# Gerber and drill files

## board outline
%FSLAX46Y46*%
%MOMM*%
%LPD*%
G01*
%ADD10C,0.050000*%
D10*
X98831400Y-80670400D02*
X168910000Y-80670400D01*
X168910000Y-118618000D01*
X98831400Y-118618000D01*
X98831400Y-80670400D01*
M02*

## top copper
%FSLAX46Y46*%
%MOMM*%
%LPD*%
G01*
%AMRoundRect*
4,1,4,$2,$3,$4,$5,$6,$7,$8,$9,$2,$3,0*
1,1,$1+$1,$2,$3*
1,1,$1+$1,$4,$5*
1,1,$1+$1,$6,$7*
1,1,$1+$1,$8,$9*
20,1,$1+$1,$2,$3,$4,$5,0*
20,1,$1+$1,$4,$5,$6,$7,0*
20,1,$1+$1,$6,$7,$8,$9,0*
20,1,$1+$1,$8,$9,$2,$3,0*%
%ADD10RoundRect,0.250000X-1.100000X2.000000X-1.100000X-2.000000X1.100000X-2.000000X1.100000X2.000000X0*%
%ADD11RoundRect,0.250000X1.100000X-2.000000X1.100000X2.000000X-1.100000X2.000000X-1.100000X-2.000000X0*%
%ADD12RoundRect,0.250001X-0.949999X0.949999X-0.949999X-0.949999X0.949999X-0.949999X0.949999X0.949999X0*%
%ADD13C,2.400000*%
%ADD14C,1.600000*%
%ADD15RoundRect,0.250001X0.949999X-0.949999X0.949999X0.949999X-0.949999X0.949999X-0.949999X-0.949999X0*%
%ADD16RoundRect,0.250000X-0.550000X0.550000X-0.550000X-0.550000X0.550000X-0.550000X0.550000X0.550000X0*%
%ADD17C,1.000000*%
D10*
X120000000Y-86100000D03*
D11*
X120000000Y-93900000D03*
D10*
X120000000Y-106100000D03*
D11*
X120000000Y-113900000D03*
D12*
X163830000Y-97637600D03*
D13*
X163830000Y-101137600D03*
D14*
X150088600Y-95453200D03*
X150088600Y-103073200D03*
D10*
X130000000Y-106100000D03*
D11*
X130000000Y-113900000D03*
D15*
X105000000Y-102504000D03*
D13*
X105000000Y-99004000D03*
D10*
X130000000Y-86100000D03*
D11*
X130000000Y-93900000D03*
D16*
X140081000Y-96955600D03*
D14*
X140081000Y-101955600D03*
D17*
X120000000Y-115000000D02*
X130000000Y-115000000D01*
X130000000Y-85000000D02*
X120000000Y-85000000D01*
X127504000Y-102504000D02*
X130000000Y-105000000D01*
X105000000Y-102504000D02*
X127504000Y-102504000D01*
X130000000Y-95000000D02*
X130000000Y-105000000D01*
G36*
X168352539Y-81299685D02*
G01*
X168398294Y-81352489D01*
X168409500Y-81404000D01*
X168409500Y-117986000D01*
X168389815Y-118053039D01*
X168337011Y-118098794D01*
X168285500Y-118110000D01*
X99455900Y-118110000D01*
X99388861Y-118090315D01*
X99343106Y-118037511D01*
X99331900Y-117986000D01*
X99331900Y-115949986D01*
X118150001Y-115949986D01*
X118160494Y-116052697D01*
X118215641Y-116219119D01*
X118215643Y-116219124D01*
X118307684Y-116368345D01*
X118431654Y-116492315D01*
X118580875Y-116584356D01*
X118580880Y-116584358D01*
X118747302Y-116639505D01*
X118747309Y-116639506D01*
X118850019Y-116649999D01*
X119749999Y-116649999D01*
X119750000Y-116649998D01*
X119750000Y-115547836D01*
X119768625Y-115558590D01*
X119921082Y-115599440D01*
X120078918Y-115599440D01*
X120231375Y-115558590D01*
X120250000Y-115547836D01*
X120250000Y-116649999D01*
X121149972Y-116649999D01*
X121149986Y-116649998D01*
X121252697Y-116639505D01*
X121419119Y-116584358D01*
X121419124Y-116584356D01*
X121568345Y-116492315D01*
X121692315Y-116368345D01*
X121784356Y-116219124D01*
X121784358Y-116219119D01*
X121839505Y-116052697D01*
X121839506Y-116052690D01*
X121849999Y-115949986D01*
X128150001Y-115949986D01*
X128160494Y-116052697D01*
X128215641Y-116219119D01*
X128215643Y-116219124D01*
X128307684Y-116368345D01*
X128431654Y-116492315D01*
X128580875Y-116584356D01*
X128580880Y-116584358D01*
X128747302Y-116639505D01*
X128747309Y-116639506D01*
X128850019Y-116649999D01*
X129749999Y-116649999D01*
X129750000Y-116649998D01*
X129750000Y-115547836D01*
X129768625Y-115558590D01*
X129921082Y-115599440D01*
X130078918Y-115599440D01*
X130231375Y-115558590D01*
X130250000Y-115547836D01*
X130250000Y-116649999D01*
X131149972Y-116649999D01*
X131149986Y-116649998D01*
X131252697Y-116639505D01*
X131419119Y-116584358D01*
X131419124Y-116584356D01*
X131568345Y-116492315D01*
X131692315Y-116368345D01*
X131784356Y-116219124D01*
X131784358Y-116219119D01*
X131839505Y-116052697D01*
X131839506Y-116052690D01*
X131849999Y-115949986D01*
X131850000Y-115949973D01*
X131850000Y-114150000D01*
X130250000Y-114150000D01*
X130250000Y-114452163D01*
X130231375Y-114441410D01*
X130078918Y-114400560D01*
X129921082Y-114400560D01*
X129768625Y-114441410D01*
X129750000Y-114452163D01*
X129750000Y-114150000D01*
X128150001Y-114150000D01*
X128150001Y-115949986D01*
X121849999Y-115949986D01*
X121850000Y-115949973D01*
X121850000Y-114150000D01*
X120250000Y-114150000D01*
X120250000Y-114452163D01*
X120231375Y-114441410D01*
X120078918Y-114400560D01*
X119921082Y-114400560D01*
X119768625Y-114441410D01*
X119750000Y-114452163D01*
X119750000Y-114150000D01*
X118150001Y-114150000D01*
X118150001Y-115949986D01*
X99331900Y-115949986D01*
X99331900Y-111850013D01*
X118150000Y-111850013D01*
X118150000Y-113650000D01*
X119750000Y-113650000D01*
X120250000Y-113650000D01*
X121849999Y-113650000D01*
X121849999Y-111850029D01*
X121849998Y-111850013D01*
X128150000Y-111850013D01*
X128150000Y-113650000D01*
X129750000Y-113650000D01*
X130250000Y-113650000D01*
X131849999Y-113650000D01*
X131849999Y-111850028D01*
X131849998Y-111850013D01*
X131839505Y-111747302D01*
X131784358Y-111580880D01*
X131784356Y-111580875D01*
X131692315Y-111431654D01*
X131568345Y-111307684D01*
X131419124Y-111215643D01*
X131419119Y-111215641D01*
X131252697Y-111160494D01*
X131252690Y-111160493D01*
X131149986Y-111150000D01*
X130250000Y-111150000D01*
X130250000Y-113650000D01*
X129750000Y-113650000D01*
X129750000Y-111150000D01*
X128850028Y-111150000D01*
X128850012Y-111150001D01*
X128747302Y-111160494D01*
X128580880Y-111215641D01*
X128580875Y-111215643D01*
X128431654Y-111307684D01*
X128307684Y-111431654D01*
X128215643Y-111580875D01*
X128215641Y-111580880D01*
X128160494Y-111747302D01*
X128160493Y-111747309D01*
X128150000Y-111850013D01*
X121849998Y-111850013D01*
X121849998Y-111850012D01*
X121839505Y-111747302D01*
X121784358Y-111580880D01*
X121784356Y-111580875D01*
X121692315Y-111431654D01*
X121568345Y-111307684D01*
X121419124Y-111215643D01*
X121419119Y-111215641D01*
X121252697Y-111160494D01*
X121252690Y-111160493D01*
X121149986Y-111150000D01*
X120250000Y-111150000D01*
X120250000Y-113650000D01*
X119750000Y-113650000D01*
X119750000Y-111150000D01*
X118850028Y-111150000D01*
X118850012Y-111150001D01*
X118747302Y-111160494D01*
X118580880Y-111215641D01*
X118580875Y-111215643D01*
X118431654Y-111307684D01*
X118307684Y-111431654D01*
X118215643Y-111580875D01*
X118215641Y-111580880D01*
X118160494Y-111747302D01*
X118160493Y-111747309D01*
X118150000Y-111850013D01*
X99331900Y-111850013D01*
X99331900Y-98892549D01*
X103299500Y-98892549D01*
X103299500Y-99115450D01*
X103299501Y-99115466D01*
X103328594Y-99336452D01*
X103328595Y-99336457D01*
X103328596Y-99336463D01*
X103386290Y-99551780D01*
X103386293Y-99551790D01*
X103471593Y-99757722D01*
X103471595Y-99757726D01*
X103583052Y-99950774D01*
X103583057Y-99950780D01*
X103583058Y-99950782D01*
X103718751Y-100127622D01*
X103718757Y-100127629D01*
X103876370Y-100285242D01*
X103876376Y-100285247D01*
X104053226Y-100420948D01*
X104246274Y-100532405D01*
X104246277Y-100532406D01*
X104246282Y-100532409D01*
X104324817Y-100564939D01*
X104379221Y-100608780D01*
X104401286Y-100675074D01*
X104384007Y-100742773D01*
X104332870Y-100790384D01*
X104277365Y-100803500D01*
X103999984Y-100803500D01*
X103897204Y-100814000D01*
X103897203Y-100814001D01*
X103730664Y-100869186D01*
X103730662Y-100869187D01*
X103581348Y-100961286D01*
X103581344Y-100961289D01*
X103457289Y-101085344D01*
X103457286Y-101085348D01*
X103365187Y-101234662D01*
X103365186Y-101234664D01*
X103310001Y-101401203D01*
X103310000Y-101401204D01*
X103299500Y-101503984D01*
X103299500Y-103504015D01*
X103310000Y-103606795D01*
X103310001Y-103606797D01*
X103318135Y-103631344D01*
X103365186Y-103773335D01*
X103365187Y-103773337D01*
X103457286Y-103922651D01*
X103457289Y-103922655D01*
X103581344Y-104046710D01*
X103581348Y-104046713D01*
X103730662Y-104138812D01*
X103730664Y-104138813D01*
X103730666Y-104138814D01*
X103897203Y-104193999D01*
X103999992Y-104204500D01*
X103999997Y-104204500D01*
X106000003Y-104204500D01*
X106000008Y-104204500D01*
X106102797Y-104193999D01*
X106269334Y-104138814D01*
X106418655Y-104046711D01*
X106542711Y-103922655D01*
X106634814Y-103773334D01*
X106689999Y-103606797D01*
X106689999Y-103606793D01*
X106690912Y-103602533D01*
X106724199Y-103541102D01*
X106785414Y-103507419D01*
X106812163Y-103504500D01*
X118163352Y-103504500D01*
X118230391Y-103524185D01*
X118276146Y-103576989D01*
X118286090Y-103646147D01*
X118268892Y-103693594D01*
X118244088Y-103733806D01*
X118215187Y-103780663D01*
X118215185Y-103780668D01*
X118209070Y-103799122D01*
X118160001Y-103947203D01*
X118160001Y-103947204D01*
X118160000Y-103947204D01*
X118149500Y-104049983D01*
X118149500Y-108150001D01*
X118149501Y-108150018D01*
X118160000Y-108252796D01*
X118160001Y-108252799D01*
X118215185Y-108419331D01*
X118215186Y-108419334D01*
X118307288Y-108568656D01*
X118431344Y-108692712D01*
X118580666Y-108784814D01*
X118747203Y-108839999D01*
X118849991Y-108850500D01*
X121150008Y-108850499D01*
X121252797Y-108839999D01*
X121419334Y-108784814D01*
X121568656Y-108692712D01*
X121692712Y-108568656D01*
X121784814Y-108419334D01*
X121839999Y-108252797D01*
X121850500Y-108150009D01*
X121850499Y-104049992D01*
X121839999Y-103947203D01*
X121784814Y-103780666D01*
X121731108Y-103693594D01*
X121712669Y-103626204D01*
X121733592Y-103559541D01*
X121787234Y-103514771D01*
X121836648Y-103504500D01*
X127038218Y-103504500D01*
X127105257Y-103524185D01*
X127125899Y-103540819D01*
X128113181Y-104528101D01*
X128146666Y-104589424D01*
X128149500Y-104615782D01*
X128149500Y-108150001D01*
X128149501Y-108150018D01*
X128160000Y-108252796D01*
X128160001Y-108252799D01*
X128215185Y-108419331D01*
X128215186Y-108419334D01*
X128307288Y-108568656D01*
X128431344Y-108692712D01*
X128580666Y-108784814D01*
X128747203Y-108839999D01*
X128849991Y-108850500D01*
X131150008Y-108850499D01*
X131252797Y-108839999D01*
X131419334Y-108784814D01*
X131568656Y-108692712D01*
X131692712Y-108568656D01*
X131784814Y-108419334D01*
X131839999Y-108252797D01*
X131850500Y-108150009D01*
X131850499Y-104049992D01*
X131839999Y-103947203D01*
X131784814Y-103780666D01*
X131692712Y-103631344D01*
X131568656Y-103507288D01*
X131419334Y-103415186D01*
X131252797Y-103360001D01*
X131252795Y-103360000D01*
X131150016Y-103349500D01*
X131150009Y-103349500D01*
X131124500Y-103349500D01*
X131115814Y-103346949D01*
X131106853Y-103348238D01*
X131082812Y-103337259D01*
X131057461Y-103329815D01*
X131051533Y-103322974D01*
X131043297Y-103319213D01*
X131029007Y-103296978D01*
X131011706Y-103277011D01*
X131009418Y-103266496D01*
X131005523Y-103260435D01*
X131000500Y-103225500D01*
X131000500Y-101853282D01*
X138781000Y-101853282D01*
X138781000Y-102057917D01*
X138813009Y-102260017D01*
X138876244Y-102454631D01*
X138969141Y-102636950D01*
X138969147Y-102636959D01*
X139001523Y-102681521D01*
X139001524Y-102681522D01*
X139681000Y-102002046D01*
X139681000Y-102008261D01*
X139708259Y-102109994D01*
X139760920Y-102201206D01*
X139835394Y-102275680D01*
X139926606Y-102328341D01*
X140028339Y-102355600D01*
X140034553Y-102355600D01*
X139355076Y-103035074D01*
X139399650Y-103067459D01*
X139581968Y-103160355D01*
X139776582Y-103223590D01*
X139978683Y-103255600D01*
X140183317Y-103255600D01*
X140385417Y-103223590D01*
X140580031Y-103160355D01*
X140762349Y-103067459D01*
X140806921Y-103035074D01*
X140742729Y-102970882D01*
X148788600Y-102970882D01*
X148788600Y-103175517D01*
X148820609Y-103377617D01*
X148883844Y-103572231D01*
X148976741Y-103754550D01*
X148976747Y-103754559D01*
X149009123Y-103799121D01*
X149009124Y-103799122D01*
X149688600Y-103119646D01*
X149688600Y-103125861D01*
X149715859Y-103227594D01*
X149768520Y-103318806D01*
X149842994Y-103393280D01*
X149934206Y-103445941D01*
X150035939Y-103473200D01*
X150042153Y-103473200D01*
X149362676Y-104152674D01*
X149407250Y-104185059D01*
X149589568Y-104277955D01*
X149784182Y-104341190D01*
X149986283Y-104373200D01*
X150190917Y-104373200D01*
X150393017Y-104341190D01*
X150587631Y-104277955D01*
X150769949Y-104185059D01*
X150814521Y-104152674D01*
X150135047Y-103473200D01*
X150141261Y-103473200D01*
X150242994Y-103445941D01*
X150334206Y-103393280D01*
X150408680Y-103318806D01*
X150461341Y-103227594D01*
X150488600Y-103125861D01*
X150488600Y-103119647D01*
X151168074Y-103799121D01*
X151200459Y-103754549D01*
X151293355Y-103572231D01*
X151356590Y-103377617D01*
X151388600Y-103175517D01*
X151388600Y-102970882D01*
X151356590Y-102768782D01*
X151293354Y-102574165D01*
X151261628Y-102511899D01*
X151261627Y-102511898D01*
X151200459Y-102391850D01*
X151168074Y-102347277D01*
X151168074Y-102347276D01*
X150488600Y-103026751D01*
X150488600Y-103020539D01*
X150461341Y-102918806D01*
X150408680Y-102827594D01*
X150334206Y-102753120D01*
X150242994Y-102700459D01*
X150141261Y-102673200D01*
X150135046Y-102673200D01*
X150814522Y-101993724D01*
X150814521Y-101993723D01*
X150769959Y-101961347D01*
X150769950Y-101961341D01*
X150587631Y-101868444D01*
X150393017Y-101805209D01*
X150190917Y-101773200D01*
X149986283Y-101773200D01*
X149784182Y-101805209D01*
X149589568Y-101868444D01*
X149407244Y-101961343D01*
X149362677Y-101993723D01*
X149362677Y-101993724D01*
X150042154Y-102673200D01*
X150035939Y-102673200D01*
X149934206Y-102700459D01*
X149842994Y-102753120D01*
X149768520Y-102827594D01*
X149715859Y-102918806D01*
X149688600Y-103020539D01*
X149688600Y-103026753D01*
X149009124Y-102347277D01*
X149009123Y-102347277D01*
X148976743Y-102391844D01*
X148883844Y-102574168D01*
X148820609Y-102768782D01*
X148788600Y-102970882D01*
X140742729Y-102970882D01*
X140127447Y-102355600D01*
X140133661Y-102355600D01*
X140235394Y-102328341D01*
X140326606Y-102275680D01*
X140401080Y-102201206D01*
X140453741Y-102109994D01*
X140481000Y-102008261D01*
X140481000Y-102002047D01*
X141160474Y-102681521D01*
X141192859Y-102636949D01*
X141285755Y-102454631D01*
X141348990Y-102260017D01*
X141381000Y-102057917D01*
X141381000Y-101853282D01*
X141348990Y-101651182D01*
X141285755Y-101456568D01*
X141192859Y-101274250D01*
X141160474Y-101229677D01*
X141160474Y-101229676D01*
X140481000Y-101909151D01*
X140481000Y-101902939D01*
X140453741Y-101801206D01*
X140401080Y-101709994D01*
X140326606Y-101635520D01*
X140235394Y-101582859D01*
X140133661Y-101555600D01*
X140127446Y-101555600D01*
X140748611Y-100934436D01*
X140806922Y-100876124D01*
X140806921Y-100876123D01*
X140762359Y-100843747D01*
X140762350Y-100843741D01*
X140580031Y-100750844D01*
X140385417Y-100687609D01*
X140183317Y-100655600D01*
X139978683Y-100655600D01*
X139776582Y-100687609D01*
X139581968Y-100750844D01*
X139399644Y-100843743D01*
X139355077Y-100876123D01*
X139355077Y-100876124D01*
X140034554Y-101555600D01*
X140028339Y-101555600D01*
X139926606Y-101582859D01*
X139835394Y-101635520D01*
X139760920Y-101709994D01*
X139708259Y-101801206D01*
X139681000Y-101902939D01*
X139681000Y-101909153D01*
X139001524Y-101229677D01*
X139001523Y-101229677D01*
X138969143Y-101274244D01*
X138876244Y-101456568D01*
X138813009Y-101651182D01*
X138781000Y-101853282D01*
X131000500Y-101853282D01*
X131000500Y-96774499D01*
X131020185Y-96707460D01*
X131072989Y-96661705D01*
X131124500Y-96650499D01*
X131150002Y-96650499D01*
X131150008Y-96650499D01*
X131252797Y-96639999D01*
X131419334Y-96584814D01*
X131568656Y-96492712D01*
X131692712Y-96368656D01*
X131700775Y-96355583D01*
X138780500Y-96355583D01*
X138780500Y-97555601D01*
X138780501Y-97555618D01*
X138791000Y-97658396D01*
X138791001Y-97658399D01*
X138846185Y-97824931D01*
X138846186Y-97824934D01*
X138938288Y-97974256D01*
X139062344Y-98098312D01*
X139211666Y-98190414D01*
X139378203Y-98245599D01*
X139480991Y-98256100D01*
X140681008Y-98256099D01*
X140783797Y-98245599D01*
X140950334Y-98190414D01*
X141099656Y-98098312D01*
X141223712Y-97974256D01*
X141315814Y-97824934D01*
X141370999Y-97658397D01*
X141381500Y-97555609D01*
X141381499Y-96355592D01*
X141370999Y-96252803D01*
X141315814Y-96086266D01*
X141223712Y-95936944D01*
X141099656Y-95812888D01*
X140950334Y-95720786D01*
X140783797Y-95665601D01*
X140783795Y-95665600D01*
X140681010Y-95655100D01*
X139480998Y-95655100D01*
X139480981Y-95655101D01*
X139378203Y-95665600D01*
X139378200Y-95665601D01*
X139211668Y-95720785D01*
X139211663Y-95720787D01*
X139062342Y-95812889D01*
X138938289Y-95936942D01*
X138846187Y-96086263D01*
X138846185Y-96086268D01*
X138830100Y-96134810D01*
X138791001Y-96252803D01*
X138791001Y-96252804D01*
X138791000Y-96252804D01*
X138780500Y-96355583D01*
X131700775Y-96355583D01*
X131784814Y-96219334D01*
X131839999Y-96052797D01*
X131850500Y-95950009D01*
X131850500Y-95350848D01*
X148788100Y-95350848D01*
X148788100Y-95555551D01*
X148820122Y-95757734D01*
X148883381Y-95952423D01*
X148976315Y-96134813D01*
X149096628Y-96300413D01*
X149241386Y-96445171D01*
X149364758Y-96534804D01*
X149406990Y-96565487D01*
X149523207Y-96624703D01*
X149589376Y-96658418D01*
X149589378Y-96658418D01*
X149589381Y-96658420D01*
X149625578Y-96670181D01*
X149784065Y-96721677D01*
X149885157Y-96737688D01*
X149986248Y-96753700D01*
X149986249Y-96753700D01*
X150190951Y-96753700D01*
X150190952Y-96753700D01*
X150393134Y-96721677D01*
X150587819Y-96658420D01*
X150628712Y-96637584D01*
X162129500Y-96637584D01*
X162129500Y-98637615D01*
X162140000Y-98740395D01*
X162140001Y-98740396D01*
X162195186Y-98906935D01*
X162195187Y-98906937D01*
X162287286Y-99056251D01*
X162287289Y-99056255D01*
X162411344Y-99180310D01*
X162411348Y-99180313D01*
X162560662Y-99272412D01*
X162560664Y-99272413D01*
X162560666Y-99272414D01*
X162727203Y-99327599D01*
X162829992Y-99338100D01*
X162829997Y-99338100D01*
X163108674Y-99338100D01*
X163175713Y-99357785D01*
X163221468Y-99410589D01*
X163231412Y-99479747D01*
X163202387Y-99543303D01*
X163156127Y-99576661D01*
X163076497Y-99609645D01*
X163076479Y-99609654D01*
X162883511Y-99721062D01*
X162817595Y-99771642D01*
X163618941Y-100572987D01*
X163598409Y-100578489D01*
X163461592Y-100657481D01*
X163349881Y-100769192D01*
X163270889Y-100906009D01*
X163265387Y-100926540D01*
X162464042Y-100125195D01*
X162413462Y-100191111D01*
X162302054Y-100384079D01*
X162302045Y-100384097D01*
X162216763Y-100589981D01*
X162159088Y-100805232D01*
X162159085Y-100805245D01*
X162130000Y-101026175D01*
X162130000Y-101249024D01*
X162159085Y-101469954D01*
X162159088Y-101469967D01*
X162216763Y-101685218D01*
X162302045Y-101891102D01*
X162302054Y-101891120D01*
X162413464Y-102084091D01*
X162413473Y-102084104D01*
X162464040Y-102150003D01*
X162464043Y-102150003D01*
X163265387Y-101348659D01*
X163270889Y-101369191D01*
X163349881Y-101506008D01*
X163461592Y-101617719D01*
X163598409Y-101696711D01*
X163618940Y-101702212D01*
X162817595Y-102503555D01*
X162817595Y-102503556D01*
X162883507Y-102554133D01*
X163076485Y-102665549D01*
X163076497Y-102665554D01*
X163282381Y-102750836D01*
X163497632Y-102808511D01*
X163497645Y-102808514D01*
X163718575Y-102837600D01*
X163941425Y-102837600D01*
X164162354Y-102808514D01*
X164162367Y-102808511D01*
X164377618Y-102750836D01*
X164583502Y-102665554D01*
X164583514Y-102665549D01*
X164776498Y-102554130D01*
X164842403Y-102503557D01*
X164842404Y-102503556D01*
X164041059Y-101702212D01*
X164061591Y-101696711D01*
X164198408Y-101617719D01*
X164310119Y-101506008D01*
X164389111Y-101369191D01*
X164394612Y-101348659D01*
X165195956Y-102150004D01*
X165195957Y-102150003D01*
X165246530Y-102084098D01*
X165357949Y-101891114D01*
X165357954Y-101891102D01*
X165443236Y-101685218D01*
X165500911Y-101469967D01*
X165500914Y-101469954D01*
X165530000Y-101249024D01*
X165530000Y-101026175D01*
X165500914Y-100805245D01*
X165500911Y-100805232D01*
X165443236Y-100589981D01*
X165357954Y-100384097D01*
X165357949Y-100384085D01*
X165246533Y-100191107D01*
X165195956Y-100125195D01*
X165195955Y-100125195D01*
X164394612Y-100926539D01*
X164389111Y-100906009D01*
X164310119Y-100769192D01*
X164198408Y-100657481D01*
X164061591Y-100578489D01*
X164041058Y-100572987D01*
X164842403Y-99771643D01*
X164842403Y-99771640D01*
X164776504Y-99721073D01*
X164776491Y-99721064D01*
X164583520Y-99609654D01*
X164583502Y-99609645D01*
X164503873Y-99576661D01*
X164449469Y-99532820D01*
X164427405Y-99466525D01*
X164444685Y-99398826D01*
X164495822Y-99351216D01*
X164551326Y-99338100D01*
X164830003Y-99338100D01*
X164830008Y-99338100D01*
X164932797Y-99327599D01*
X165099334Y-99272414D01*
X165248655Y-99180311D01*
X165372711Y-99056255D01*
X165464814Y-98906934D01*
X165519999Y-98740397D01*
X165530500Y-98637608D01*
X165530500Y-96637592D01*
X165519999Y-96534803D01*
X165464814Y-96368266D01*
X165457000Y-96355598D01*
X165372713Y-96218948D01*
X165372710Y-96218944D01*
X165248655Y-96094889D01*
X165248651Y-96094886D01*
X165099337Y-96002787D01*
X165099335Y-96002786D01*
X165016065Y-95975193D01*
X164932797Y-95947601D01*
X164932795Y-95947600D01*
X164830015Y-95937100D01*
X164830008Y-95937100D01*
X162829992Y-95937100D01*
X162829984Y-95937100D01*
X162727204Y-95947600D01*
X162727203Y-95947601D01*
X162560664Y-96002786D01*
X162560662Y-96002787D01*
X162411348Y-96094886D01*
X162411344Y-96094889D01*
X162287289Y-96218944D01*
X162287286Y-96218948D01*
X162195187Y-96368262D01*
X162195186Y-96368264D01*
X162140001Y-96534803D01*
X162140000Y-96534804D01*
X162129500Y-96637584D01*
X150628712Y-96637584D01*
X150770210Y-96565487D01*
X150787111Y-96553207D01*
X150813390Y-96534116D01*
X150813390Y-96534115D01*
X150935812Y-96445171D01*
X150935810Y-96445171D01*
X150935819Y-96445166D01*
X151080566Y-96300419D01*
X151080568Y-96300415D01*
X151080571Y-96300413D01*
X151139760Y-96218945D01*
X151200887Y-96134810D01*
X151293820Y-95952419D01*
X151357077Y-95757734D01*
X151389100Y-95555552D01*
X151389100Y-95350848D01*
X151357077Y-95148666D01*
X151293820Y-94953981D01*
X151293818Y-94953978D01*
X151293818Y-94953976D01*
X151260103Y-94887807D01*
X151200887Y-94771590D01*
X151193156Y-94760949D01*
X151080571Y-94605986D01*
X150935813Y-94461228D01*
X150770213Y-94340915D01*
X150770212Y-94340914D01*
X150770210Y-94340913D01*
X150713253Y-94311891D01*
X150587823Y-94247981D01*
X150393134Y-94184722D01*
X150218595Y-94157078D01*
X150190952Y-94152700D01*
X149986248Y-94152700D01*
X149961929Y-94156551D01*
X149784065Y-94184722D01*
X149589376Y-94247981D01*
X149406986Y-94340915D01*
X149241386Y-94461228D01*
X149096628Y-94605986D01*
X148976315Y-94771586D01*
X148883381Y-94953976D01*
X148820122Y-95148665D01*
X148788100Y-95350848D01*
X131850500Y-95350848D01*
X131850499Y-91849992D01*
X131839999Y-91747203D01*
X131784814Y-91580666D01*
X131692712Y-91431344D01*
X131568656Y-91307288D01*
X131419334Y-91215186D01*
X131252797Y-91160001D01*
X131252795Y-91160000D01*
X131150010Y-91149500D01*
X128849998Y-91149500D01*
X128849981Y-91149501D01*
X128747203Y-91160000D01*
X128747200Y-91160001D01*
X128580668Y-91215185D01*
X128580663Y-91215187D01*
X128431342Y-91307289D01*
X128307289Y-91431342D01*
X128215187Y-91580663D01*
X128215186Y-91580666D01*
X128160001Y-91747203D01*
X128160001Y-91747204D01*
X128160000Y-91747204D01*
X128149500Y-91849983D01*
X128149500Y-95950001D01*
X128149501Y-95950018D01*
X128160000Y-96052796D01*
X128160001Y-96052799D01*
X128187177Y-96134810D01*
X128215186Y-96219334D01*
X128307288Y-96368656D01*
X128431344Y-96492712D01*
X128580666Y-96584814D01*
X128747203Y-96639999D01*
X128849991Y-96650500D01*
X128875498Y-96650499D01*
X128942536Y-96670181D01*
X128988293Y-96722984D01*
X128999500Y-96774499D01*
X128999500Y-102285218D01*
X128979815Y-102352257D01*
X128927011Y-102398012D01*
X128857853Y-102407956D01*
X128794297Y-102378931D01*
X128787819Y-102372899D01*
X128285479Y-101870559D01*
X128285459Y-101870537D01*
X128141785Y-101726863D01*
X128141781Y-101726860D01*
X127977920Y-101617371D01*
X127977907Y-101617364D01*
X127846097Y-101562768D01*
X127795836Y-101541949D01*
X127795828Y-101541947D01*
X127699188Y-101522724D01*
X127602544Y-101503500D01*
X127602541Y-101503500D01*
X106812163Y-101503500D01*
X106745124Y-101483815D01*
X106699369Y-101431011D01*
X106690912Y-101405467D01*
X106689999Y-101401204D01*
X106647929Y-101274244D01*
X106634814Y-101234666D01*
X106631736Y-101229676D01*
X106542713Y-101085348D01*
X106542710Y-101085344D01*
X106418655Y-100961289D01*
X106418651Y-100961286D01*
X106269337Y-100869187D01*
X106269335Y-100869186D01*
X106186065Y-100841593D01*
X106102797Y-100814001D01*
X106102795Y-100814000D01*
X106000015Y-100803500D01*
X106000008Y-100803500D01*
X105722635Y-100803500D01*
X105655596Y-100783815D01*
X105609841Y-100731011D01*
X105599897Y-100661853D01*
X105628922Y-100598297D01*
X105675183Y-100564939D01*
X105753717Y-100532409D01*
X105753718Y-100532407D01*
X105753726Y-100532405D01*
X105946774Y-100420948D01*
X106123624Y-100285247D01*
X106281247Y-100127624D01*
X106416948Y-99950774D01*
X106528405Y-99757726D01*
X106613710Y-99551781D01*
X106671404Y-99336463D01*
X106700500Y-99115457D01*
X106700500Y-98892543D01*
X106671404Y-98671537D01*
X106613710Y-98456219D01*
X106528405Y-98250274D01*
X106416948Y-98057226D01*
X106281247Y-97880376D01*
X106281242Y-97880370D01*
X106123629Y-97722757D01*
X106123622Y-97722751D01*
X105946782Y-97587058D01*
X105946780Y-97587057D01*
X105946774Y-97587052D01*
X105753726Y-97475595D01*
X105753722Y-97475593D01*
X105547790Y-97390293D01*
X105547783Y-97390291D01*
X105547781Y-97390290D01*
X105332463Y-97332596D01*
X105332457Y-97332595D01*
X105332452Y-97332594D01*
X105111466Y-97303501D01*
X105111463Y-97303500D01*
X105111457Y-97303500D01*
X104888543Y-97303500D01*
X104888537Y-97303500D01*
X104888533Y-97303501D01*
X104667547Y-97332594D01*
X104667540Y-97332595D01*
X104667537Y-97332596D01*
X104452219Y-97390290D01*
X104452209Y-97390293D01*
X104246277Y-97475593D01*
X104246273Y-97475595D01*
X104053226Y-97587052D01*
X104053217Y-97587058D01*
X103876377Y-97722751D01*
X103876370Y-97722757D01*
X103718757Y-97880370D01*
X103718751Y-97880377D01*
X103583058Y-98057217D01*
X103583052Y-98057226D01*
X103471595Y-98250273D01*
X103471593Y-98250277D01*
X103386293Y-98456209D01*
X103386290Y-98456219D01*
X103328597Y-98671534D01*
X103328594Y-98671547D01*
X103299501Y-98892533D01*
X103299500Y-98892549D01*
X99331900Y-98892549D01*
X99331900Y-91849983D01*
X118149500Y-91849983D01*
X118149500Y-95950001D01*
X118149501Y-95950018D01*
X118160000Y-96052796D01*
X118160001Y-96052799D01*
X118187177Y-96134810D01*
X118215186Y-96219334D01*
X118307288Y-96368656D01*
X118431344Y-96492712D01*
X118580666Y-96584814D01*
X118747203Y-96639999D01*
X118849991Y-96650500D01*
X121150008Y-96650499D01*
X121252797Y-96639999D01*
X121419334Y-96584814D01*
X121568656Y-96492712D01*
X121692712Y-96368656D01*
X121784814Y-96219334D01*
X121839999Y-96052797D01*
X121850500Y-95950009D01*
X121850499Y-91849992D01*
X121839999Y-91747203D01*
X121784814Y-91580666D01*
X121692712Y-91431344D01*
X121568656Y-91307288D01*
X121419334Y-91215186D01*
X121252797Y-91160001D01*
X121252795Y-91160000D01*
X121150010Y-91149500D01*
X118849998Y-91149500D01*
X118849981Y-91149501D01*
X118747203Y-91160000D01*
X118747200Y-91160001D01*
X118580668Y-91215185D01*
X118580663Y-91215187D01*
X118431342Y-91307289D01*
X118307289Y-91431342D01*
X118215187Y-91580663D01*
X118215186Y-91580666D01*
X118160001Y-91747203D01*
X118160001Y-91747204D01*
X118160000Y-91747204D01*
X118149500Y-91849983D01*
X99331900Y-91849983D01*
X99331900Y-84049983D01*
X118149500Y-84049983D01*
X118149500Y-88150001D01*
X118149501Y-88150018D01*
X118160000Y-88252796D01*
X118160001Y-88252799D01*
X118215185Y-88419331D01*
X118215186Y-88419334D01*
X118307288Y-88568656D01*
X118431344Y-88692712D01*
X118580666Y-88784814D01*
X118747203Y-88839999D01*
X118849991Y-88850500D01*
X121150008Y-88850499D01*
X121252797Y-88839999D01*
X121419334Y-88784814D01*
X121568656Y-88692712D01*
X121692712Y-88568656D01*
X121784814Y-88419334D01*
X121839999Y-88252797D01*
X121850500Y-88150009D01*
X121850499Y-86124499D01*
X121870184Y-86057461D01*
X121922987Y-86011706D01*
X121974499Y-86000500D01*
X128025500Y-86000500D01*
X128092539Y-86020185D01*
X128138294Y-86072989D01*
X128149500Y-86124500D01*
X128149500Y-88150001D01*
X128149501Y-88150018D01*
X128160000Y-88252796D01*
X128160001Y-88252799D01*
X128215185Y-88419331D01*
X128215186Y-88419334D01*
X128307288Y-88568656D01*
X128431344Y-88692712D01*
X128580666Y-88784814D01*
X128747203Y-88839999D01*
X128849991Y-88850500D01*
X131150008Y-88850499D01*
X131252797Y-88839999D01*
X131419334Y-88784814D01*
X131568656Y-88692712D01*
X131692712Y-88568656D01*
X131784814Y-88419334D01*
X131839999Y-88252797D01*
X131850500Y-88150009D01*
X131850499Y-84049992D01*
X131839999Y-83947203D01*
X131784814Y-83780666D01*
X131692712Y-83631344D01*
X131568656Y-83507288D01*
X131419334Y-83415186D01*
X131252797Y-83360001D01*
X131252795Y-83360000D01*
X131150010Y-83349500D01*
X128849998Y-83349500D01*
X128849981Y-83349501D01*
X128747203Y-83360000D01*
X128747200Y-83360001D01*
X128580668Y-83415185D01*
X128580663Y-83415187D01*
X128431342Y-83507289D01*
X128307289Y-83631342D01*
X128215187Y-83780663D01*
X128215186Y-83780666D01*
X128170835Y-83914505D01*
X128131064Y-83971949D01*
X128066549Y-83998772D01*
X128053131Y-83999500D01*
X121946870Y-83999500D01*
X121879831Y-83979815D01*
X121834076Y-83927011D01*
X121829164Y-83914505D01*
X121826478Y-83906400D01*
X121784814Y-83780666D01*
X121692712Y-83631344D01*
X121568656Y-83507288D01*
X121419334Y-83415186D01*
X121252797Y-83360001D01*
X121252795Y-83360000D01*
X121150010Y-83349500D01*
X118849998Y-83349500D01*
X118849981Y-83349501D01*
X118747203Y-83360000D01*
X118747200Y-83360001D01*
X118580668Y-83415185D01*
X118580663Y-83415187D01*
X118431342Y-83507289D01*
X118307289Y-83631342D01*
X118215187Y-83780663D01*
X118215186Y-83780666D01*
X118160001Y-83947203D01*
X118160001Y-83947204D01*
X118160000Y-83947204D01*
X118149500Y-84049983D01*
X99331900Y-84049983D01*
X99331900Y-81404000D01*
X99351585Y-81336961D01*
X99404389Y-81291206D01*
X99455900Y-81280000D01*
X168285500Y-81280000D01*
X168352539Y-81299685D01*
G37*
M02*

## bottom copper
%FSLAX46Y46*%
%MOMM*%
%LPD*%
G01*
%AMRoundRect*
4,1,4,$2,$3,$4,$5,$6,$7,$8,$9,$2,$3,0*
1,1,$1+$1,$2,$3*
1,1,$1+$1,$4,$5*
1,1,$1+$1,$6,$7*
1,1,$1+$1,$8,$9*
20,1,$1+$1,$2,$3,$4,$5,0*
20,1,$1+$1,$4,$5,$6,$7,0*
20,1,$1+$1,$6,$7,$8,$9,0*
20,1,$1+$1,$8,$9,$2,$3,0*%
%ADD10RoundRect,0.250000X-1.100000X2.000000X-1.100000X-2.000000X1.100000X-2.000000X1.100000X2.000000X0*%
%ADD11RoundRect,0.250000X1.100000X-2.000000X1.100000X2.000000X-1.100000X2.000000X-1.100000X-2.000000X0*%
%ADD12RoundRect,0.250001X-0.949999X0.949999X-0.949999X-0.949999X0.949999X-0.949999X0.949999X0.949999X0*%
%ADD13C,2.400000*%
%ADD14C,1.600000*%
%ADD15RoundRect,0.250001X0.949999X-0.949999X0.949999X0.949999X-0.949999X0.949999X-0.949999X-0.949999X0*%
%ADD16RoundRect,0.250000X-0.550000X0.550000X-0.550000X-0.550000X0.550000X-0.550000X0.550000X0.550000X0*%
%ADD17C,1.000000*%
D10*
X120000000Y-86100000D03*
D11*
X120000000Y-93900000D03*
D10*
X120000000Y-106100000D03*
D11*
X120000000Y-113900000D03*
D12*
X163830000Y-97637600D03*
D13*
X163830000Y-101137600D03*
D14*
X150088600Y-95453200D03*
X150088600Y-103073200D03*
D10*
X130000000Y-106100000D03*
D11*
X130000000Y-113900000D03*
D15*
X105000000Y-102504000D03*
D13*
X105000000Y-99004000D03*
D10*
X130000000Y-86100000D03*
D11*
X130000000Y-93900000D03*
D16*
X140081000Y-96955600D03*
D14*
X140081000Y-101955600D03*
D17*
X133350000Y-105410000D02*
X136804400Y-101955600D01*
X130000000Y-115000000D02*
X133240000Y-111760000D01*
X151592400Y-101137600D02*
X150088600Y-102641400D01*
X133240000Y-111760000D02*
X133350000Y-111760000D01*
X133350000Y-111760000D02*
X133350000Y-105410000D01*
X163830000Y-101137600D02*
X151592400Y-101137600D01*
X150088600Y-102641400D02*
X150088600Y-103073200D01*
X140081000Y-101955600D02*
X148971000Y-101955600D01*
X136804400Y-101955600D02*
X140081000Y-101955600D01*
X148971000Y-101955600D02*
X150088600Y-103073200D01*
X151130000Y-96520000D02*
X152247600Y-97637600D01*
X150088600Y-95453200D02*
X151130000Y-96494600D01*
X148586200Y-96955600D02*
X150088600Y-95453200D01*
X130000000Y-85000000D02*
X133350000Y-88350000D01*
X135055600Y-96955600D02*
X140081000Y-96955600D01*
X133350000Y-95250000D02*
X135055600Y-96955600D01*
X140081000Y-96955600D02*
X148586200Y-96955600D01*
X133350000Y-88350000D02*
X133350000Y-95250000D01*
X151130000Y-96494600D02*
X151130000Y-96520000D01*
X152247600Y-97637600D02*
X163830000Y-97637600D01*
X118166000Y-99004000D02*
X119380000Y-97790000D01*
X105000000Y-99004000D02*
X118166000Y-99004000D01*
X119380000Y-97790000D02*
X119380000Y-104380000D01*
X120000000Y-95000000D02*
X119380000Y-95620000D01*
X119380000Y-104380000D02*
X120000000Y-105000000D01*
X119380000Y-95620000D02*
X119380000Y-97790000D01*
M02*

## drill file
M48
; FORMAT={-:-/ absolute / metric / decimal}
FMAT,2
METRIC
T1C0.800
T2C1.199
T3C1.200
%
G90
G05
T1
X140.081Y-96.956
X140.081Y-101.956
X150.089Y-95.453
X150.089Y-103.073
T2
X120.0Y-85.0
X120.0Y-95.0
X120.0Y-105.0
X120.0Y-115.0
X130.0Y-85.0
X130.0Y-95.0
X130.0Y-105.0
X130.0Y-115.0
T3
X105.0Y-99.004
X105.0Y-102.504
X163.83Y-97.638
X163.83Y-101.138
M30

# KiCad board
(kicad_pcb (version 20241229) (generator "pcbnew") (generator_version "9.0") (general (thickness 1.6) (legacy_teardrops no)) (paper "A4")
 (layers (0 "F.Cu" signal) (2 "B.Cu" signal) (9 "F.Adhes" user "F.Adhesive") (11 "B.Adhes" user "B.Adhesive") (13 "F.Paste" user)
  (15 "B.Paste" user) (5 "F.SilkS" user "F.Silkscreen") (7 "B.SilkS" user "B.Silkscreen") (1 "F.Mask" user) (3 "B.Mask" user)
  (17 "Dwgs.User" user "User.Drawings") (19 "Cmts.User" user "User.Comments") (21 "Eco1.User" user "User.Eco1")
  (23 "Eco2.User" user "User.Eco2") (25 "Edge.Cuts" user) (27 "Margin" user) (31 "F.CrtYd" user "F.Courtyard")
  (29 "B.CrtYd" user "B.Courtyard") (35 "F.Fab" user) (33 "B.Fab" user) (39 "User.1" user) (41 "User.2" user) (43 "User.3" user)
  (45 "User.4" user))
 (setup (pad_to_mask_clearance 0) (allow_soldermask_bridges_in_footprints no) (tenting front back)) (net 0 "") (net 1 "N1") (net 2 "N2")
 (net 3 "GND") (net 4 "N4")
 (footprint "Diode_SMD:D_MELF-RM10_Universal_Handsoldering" (layer "F.Cu") (at 120 90 -90)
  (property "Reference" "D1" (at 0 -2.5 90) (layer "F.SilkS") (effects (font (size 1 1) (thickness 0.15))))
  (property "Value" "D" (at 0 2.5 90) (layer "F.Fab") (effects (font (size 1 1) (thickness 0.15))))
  (pad "1" thru_hole roundrect (at -5 0 270) (size 4.5 2.7) (drill 1.19888 (offset 1.1 0)) (layers "*.Cu" "*.Mask")
   (remove_unused_layers no) (roundrect_rratio 0.0925925926) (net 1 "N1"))
  (pad "2" thru_hole roundrect (at 5 0 90) (size 4.5 2.7) (drill 1.19888 (offset 1.1 0)) (layers "*.Cu" "*.Mask") (remove_unused_layers no)
   (roundrect_rratio 0.0925925926) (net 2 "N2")))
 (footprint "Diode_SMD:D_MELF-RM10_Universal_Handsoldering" (layer "F.Cu") (at 120 110 -90)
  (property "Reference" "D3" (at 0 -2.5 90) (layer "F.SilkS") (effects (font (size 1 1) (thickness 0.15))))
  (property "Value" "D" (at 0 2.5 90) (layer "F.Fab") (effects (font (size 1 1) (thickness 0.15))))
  (pad "1" thru_hole roundrect (at -5 0 270) (size 4.5 2.7) (drill 1.19888 (offset 1.1 0)) (layers "*.Cu" "*.Mask")
   (remove_unused_layers no) (roundrect_rratio 0.0925925926) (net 2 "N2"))
  (pad "2" thru_hole roundrect (at 5 0 90) (size 4.5 2.7) (drill 1.19888 (offset 1.1 0)) (layers "*.Cu" "*.Mask") (remove_unused_layers no)
   (roundrect_rratio 0.0925925926) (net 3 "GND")))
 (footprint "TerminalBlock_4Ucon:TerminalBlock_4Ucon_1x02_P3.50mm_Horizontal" (layer "F.Cu") (at 163.83 97.6376 -90)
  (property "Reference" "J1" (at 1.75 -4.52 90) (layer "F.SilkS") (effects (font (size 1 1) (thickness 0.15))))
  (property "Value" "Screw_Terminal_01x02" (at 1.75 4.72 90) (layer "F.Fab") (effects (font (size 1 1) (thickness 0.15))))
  (pad "1" thru_hole roundrect (at 0 0 270) (size 2.4 2.4) (drill 1.2) (layers "*.Cu" "*.Mask") (remove_unused_layers no)
   (roundrect_rratio 0.104167) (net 1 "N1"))
  (pad "2" thru_hole circle (at 3.5 0 270) (size 2.4 2.4) (drill 1.2) (layers "*.Cu" "*.Mask") (remove_unused_layers no) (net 3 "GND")))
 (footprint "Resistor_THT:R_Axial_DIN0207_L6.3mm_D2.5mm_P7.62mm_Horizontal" (layer "F.Cu") (at 150.0886 95.4532 -90)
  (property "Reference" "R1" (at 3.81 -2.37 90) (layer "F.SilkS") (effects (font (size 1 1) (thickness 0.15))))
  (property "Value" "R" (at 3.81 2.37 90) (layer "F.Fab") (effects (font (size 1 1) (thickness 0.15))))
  (pad "1" thru_hole circle (at 0 0 270) (size 1.6 1.6) (drill 0.8) (layers "*.Cu" "*.Mask") (remove_unused_layers no) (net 1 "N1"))
  (pad "2" thru_hole circle (at 7.62 0 270) (size 1.6 1.6) (drill 0.8) (layers "*.Cu" "*.Mask") (remove_unused_layers no) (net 3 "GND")))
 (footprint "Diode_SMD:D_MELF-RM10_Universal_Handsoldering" (layer "F.Cu") (at 130 110 -90)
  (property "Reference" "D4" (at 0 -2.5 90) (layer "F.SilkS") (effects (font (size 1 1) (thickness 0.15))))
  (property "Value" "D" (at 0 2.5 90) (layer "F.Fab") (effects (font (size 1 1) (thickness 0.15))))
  (pad "1" thru_hole roundrect (at -5 0 270) (size 4.5 2.7) (drill 1.19888 (offset 1.1 0)) (layers "*.Cu" "*.Mask")
   (remove_unused_layers no) (roundrect_rratio 0.0925925926) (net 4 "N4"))
  (pad "2" thru_hole roundrect (at 5 0 90) (size 4.5 2.7) (drill 1.19888 (offset 1.1 0)) (layers "*.Cu" "*.Mask") (remove_unused_layers no)
   (roundrect_rratio 0.0925925926) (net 3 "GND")))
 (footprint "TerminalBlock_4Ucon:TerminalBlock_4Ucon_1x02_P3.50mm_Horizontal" (layer "F.Cu") (at 105 102.504 90)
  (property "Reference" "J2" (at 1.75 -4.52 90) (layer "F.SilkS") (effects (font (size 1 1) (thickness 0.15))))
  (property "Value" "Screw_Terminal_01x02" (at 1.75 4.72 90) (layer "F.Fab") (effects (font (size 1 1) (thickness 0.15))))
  (pad "1" thru_hole roundrect (at 0 0 90) (size 2.4 2.4) (drill 1.2) (layers "*.Cu" "*.Mask") (remove_unused_layers no)
   (roundrect_rratio 0.104167) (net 4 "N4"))
  (pad "2" thru_hole circle (at 3.5 0 90) (size 2.4 2.4) (drill 1.2) (layers "*.Cu" "*.Mask") (remove_unused_layers no) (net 2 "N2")))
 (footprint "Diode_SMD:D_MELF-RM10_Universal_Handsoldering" (layer "F.Cu") (at 130 90 -90)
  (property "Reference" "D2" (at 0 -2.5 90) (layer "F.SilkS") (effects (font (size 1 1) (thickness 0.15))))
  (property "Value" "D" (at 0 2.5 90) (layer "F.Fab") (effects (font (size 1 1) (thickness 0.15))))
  (pad "1" thru_hole roundrect (at -5 0 270) (size 4.5 2.7) (drill 1.19888 (offset 1.1 0)) (layers "*.Cu" "*.Mask")
   (remove_unused_layers no) (roundrect_rratio 0.0925925926) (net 1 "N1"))
  (pad "2" thru_hole roundrect (at 5 0 90) (size 4.5 2.7) (drill 1.19888 (offset 1.1 0)) (layers "*.Cu" "*.Mask") (remove_unused_layers no)
   (roundrect_rratio 0.0925925926) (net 4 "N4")))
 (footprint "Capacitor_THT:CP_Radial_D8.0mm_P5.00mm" (layer "F.Cu") (at 140.081 96.9556 -90)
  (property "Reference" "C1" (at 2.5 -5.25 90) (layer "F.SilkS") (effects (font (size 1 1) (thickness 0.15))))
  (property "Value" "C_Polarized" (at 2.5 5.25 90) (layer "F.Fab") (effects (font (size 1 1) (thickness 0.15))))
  (pad "1" thru_hole roundrect (at 0 0 270) (size 1.6 1.6) (drill 0.8) (layers "*.Cu" "*.Mask") (remove_unused_layers no)
   (roundrect_rratio 0.15625) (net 1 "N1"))
  (pad "2" thru_hole circle (at 5 0 270) (size 1.6 1.6) (drill 0.8) (layers "*.Cu" "*.Mask") (remove_unused_layers no) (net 3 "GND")))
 (gr_rect (start 98.8314 80.6704) (end 168.91 118.618) (stroke (width 0.05) (type default)) (fill no) (layer "Edge.Cuts"))
 (segment (start 120 115) (end 130 115) (width 1) (layer "F.Cu") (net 3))
 (segment (start 133.35 105.41) (end 136.8044 101.9556) (width 1) (layer "B.Cu") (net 3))
 (segment (start 130 115) (end 133.24 111.76) (width 1) (layer "B.Cu") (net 3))
 (segment (start 151.5924 101.1376) (end 150.0886 102.6414) (width 1) (layer "B.Cu") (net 3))
 (segment (start 133.24 111.76) (end 133.35 111.76) (width 1) (layer "B.Cu") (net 3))
 (segment (start 133.35 111.76) (end 133.35 105.41) (width 1) (layer "B.Cu") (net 3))
 (segment (start 163.83 101.1376) (end 151.5924 101.1376) (width 1) (layer "B.Cu") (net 3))
 (segment (start 150.0886 102.6414) (end 150.0886 103.0732) (width 1) (layer "B.Cu") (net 3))
 (segment (start 140.081 101.9556) (end 148.971 101.9556) (width 1) (layer "B.Cu") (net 3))
 (segment (start 136.8044 101.9556) (end 140.081 101.9556) (width 1) (layer "B.Cu") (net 3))
 (segment (start 148.971 101.9556) (end 150.0886 103.0732) (width 1) (layer "B.Cu") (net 3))
 (segment (start 130 85) (end 120 85) (width 1) (layer "F.Cu") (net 1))
 (segment (start 151.13 96.52) (end 152.2476 97.6376) (width 1) (layer "B.Cu") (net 1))
 (segment (start 150.0886 95.4532) (end 151.13 96.4946) (width 1) (layer "B.Cu") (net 1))
 (segment (start 148.5862 96.9556) (end 150.0886 95.4532) (width 1) (layer "B.Cu") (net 1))
 (segment (start 130 85) (end 133.35 88.35) (width 1) (layer "B.Cu") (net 1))
 (segment (start 135.0556 96.9556) (end 140.081 96.9556) (width 1) (layer "B.Cu") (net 1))
 (segment (start 133.35 95.25) (end 135.0556 96.9556) (width 1) (layer "B.Cu") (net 1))
 (segment (start 140.081 96.9556) (end 148.5862 96.9556) (width 1) (layer "B.Cu") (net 1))
 (segment (start 133.35 88.35) (end 133.35 95.25) (width 1) (layer "B.Cu") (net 1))
 (segment (start 151.13 96.4946) (end 151.13 96.52) (width 1) (layer "B.Cu") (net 1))
 (segment (start 152.2476 97.6376) (end 163.83 97.6376) (width 1) (layer "B.Cu") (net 1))
 (segment (start 118.166 99.004) (end 119.38 97.79) (width 1) (layer "B.Cu") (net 2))
 (segment (start 105 99.004) (end 118.166 99.004) (width 1) (layer "B.Cu") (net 2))
 (segment (start 119.38 97.79) (end 119.38 104.38) (width 1) (layer "B.Cu") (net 2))
 (segment (start 120 95) (end 119.38 95.62) (width 1) (layer "B.Cu") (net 2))
 (segment (start 119.38 104.38) (end 120 105) (width 1) (layer "B.Cu") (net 2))
 (segment (start 119.38 95.62) (end 119.38 97.79) (width 1) (layer "B.Cu") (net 2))
 (segment (start 127.504 102.504) (end 130 105) (width 1) (layer "F.Cu") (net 4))
 (segment (start 105 102.504) (end 127.504 102.504) (width 1) (layer "F.Cu") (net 4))
 (segment (start 130 95) (end 130 105) (width 1) (layer "F.Cu") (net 4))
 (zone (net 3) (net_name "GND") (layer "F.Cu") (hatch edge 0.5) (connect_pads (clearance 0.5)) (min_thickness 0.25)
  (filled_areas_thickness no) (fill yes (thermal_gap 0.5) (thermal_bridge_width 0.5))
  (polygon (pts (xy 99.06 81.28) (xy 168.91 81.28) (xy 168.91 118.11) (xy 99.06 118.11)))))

